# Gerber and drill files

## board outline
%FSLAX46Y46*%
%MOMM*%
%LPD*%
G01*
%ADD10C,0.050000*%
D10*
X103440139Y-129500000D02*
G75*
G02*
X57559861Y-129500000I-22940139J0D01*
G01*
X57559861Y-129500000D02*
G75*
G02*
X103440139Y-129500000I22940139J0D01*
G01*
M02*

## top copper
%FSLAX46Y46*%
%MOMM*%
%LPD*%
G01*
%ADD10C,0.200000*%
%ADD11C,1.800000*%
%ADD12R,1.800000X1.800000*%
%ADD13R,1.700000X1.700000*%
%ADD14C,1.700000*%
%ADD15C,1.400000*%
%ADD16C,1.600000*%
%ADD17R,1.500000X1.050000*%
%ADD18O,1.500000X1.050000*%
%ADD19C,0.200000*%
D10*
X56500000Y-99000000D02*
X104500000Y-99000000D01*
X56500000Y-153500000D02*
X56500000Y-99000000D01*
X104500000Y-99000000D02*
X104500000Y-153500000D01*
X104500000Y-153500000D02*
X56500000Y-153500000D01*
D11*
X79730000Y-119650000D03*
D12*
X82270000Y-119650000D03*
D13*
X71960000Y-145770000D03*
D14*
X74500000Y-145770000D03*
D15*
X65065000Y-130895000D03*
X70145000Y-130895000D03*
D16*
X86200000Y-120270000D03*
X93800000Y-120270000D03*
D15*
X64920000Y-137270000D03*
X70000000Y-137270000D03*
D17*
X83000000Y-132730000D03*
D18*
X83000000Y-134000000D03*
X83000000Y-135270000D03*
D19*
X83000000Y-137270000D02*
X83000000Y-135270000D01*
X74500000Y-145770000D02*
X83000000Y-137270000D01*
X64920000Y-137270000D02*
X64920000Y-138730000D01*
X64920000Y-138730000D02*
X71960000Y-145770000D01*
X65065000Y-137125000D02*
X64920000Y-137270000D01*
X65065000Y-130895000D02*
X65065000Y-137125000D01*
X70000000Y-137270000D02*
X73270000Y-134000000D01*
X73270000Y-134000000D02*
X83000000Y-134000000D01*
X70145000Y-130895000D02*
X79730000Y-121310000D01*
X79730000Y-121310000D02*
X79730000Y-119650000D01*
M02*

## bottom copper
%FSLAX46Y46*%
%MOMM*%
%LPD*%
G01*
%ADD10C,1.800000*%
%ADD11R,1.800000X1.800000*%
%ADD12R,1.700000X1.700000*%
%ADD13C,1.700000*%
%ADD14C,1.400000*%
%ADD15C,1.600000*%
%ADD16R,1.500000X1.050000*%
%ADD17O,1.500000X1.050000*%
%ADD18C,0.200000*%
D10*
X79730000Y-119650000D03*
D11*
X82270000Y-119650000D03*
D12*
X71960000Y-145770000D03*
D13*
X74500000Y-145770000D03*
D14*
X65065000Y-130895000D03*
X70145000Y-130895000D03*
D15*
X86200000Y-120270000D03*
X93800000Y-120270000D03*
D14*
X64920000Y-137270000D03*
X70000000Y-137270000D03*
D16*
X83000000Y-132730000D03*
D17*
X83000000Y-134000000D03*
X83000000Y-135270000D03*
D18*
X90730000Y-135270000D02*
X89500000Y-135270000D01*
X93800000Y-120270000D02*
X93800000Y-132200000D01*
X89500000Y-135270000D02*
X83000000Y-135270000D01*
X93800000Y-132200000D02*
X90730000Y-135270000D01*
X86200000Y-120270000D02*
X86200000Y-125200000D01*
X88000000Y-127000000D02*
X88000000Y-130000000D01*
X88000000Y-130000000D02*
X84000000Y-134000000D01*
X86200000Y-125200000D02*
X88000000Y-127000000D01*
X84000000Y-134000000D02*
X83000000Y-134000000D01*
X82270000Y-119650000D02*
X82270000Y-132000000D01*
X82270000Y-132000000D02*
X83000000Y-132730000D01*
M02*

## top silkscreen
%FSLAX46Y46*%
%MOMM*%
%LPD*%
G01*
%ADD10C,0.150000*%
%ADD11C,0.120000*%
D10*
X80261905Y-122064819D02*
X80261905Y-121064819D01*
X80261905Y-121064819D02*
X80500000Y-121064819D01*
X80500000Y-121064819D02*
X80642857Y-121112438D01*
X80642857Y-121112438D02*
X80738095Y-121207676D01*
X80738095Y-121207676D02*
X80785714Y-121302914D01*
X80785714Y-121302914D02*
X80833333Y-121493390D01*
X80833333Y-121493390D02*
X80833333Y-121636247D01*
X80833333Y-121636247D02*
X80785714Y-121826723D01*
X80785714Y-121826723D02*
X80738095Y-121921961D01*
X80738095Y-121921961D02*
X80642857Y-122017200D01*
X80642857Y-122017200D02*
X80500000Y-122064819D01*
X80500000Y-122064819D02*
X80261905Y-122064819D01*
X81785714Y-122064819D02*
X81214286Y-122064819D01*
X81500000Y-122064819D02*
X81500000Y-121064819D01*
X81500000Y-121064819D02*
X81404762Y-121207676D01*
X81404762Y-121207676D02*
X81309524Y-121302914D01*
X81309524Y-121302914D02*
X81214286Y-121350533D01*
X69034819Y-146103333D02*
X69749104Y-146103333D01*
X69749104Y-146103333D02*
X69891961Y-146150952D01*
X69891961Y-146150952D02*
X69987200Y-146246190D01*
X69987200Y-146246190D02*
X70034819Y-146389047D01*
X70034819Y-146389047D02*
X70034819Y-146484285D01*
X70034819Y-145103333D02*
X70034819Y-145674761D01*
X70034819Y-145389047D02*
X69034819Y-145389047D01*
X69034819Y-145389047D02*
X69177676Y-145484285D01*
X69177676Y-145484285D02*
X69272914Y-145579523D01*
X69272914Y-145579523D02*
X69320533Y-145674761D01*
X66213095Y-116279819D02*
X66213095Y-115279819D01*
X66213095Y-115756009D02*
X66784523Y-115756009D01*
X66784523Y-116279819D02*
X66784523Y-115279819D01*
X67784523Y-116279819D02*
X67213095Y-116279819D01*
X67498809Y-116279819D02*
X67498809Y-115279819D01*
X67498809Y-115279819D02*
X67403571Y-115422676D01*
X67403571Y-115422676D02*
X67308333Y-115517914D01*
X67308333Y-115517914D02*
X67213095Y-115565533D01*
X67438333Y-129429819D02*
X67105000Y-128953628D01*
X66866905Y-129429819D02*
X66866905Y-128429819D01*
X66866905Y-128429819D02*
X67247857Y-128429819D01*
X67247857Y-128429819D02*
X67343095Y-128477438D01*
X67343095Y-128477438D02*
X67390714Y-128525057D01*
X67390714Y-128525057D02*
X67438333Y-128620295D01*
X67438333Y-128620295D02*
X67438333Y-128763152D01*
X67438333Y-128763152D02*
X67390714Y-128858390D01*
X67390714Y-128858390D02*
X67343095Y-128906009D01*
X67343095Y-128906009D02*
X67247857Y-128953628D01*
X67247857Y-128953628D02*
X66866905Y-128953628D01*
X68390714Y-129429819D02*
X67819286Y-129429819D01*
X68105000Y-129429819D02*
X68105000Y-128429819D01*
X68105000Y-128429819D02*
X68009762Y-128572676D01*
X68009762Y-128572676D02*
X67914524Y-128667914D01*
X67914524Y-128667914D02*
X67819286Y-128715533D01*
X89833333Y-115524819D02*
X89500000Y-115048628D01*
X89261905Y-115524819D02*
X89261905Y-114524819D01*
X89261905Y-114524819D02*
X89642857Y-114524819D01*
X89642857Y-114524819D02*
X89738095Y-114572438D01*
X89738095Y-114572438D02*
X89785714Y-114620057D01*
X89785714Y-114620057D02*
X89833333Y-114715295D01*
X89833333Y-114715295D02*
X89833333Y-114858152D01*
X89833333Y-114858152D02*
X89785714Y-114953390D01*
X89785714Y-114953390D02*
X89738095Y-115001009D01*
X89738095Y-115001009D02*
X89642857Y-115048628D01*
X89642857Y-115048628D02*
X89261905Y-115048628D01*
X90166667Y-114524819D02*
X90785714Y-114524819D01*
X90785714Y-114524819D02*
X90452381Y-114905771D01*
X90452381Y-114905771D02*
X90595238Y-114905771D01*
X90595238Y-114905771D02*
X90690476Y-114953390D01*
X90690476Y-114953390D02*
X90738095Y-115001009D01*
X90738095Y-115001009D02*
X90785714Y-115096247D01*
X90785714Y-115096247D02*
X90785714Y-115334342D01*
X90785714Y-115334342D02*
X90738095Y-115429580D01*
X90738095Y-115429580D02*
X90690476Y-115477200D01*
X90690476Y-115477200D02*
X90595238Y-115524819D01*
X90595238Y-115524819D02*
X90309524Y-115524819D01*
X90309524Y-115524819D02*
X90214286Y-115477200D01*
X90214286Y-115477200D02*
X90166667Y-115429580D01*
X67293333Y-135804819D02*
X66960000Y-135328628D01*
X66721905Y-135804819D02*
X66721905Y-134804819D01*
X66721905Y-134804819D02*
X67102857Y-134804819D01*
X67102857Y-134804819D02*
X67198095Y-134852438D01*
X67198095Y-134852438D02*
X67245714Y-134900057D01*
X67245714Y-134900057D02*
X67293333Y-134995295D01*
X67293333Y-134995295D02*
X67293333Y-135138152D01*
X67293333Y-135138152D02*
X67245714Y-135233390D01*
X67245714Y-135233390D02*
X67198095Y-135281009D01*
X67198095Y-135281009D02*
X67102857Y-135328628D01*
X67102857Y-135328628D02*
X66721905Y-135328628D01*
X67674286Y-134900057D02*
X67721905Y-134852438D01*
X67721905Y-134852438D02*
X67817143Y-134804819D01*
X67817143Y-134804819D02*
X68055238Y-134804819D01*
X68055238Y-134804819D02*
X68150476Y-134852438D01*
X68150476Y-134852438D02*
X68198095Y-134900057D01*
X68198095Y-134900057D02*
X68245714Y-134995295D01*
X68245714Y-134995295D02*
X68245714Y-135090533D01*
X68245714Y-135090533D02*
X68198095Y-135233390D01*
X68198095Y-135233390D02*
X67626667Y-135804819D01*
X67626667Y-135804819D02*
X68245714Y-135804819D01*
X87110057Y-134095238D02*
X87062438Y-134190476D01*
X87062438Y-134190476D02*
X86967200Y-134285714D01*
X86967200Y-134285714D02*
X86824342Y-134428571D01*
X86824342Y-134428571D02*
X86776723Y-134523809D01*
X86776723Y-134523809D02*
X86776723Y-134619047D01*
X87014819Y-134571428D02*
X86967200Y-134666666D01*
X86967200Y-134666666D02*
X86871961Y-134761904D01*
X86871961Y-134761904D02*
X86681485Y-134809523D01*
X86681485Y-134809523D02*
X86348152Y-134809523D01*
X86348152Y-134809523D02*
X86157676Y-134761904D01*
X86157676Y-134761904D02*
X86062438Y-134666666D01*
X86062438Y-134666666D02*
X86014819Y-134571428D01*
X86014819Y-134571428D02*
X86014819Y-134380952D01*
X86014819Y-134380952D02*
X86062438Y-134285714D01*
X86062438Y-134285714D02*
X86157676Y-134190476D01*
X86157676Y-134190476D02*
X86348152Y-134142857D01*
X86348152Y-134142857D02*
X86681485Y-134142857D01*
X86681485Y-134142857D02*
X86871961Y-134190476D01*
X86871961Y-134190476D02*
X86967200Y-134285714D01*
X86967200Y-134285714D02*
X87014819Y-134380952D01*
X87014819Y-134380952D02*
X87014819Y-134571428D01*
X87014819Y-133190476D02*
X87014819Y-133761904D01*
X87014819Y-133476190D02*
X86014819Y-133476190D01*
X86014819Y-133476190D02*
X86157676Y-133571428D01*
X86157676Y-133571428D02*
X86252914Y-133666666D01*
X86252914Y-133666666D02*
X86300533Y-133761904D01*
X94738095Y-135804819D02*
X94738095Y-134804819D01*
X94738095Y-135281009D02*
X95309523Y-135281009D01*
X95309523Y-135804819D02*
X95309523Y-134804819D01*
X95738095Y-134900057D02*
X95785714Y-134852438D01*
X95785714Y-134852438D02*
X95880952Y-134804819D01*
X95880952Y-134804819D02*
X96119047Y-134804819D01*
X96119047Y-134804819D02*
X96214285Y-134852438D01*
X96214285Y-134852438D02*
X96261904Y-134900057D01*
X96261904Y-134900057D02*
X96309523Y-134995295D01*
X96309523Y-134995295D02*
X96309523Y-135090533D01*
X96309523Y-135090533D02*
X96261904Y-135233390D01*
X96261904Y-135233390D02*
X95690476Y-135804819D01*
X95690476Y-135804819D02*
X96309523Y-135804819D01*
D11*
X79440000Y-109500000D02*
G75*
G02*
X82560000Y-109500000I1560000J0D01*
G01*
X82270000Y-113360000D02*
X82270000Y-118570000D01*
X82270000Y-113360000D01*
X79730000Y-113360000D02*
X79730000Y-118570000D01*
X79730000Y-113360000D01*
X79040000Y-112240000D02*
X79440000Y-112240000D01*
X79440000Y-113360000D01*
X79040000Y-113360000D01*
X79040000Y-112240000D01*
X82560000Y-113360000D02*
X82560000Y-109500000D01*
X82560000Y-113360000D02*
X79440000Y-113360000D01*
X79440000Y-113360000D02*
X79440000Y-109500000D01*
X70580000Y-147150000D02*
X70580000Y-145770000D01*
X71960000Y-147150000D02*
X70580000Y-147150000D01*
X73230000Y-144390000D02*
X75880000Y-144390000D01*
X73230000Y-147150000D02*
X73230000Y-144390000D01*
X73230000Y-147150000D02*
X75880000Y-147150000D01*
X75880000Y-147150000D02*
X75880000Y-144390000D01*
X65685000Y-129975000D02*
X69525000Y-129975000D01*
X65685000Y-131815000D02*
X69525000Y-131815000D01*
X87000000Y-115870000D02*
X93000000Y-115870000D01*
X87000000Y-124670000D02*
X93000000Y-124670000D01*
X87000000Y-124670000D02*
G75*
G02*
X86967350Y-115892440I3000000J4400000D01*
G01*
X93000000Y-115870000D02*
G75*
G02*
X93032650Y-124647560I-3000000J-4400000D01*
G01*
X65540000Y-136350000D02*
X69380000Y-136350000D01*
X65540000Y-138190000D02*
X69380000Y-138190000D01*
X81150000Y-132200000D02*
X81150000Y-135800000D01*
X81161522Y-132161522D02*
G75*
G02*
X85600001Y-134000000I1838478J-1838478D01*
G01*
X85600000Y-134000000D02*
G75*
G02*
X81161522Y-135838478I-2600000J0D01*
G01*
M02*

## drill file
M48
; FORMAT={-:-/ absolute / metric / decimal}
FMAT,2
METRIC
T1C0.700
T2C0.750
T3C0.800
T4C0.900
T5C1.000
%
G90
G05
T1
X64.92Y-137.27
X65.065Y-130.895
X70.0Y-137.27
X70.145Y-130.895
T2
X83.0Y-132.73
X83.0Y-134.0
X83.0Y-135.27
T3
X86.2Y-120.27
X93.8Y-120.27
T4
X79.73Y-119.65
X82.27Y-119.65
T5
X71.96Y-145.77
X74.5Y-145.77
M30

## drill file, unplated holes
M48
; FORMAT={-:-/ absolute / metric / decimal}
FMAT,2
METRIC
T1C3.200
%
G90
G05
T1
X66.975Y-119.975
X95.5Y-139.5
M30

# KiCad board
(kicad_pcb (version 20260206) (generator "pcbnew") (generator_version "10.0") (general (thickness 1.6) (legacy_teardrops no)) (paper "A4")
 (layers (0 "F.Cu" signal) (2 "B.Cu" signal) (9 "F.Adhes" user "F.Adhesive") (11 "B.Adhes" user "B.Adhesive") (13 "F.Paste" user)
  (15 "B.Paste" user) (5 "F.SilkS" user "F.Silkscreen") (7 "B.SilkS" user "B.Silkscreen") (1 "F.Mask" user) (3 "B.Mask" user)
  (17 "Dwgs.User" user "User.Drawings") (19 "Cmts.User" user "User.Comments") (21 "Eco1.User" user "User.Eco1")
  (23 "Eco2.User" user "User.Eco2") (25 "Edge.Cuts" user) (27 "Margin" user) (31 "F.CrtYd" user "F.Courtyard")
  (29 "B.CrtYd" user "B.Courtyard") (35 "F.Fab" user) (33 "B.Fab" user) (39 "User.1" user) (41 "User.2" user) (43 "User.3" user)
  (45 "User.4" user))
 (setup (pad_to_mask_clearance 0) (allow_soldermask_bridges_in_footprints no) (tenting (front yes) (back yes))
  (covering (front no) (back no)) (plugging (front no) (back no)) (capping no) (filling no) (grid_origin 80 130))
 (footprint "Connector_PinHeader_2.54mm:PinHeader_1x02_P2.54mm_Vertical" (layer "F.Cu") (at 71.96 145.77 90)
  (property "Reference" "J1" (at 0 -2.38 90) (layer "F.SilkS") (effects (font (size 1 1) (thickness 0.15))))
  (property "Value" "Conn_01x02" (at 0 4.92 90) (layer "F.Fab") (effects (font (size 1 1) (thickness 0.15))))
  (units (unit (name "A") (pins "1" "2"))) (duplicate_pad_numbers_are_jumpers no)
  (fp_line (start -1.38 -1.38) (end 0 -1.38) (stroke (width 0.12) (type solid)) (layer "F.SilkS"))
  (fp_line (start -1.38 0) (end -1.38 -1.38) (stroke (width 0.12) (type solid)) (layer "F.SilkS"))
  (fp_line (start 1.38 1.27) (end 1.38 3.92) (stroke (width 0.12) (type solid)) (layer "F.SilkS"))
  (fp_line (start -1.38 1.27) (end 1.38 1.27) (stroke (width 0.12) (type solid)) (layer "F.SilkS"))
  (fp_line (start -1.38 1.27) (end -1.38 3.92) (stroke (width 0.12) (type solid)) (layer "F.SilkS"))
  (fp_line (start -1.38 3.92) (end 1.38 3.92) (stroke (width 0.12) (type solid)) (layer "F.SilkS"))
  (pad "1" thru_hole rect (at 0 0 90) (size 1.7 1.7) (drill 1) (layers "*.Cu" "*.Mask") (remove_unused_layers no) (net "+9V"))
  (pad "2" thru_hole circle (at 0 2.54 90) (size 1.7 1.7) (drill 1) (layers "*.Cu" "*.Mask") (remove_unused_layers no) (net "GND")))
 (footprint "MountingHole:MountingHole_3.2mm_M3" (layer "F.Cu") (at 66.975 119.975)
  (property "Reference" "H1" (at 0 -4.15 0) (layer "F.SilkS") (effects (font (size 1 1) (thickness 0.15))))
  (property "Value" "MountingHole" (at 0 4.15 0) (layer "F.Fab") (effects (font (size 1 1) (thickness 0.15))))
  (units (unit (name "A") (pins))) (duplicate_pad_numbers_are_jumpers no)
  (pad "" np_thru_hole circle (at 0 0) (size 3.2 3.2) (drill 3.2) (layers "*.Cu" "*.Mask")))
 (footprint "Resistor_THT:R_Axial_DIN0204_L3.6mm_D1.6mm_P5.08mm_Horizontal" (layer "F.Cu") (at 65.065 130.895)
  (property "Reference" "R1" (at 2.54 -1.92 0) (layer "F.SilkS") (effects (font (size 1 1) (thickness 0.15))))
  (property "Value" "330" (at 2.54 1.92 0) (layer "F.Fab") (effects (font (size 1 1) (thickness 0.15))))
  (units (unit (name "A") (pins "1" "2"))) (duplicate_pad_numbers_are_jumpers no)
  (fp_line (start 0.62 -0.92) (end 4.46 -0.92) (stroke (width 0.12) (type solid)) (layer "F.SilkS"))
  (fp_line (start 0.62 0.92) (end 4.46 0.92) (stroke (width 0.12) (type solid)) (layer "F.SilkS"))
  (pad "1" thru_hole circle (at 0 0) (size 1.4 1.4) (drill 0.7) (layers "*.Cu" "*.Mask") (remove_unused_layers no) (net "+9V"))
  (pad "2" thru_hole circle (at 5.08 0) (size 1.4 1.4) (drill 0.7) (layers "*.Cu" "*.Mask") (remove_unused_layers no) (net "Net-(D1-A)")))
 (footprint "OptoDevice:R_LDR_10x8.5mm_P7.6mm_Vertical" (layer "F.Cu") (at 86.2 120.27)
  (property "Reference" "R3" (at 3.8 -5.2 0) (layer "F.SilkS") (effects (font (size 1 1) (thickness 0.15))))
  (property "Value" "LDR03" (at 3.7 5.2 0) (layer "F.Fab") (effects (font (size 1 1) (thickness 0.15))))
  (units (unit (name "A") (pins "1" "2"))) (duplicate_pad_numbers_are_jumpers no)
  (fp_line (start 0.8 -4.4) (end 6.8 -4.4) (stroke (width 0.12) (type solid)) (layer "F.SilkS"))
  (fp_line (start 0.8 4.4) (end 6.8 4.4) (stroke (width 0.12) (type solid)) (layer "F.SilkS"))
  (fp_arc (start 0.8 4.4) (mid -1.525374 0.019809) (end 0.76735 -4.37756) (stroke (width 0.12) (type solid)) (layer "F.SilkS"))
  (fp_arc (start 6.8 -4.4) (mid 9.125374 -0.019809) (end 6.83265 4.37756) (stroke (width 0.12) (type solid)) (layer "F.SilkS"))
  (pad "1" thru_hole circle (at 0 0) (size 1.6 1.6) (drill 0.8) (layers "*.Cu" "*.Mask") (remove_unused_layers no) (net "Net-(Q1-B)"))
  (pad "2" thru_hole circle (at 7.6 0) (size 1.6 1.6) (drill 0.8) (layers "*.Cu" "*.Mask") (remove_unused_layers no) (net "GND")))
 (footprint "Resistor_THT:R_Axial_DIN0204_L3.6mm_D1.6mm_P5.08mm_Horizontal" (layer "F.Cu") (at 64.92 137.27)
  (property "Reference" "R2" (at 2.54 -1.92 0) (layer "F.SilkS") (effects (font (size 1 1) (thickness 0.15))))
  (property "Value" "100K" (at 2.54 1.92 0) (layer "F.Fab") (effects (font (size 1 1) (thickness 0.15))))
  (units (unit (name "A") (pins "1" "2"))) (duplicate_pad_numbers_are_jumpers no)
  (fp_line (start 0.62 -0.92) (end 4.46 -0.92) (stroke (width 0.12) (type solid)) (layer "F.SilkS"))
  (fp_line (start 0.62 0.92) (end 4.46 0.92) (stroke (width 0.12) (type solid)) (layer "F.SilkS"))
  (pad "1" thru_hole circle (at 0 0) (size 1.4 1.4) (drill 0.7) (layers "*.Cu" "*.Mask") (remove_unused_layers no) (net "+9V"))
  (pad "2" thru_hole circle (at 5.08 0) (size 1.4 1.4) (drill 0.7) (layers "*.Cu" "*.Mask") (remove_unused_layers no) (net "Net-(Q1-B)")))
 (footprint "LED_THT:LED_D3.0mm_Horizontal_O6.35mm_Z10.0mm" (layer "F.Cu") (at 82.27 119.65 180)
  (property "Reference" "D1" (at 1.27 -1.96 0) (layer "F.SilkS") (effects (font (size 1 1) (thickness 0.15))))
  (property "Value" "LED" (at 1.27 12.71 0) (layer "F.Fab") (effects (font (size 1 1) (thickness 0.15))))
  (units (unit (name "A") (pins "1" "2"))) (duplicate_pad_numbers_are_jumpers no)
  (fp_line (start 2.83 6.29) (end 2.83 10.15) (stroke (width 0.12) (type solid)) (layer "F.SilkS"))
  (fp_line (start -0.29 6.29) (end 2.83 6.29) (stroke (width 0.12) (type solid)) (layer "F.SilkS"))
  (fp_line (start -0.29 6.29) (end -0.29 10.15) (stroke (width 0.12) (type solid)) (layer "F.SilkS"))
  (fp_rect (start 2.83 6.29) (end 3.23 7.41) (stroke (width 0.12) (type solid)) (fill no) (layer "F.SilkS"))
  (fp_rect (start 2.54 1.08) (end 2.54 6.29) (stroke (width 0.12) (type solid)) (fill no) (layer "F.SilkS"))
  (fp_rect (start 0 1.08) (end 0 6.29) (stroke (width 0.12) (type solid)) (fill no) (layer "F.SilkS"))
  (fp_arc (start 2.83 10.15) (mid 1.27 11.71) (end -0.29 10.15) (stroke (width 0.12) (type solid)) (layer "F.SilkS"))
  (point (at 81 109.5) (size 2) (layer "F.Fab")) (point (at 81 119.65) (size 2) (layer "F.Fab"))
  (pad "1" thru_hole rect (at 0 0 180) (size 1.8 1.8) (drill 0.9) (layers "*.Cu" "*.Mask") (remove_unused_layers no) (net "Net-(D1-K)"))
  (pad "2" thru_hole circle (at 2.54 0 180) (size 1.8 1.8) (drill 0.9) (layers "*.Cu" "*.Mask") (remove_unused_layers no) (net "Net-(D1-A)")))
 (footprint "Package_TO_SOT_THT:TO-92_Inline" (layer "F.Cu") (at 83 132.73 -90)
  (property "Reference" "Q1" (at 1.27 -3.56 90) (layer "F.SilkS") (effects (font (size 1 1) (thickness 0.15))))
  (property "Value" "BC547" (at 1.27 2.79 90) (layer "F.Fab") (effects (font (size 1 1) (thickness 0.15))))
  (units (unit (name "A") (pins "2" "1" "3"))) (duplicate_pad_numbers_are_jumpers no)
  (fp_line (start -0.53 1.85) (end 3.07 1.85) (stroke (width 0.12) (type solid)) (layer "F.SilkS"))
  (fp_arc (start -0.568478 1.838478) (mid -1.132087 -0.994977) (end 1.27 -2.6) (stroke (width 0.12) (type solid)) (layer "F.SilkS"))
  (fp_arc (start 1.27 -2.6) (mid 3.672087 -0.994977) (end 3.108478 1.838478) (stroke (width 0.12) (type solid)) (layer "F.SilkS"))
  (pad "1" thru_hole rect (at 0 0 270) (size 1.05 1.5) (drill 0.75) (layers "*.Cu" "*.Mask") (remove_unused_layers no) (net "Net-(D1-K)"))
  (pad "2" thru_hole oval (at 1.27 0 270) (size 1.05 1.5) (drill 0.75) (layers "*.Cu" "*.Mask") (remove_unused_layers no) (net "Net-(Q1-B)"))
  (pad "3" thru_hole oval (at 2.54 0 270) (size 1.05 1.5) (drill 0.75) (layers "*.Cu" "*.Mask") (remove_unused_layers no) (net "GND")))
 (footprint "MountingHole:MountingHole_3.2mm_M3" (layer "F.Cu") (at 95.5 139.5)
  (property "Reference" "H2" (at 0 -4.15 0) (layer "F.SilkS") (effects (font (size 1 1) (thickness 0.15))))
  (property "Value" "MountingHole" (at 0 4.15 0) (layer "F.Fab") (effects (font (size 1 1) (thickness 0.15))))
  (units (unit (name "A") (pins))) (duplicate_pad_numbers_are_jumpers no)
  (pad "" np_thru_hole circle (at 0 0) (size 3.2 3.2) (drill 3.2) (layers "*.Cu" "*.Mask")))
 (gr_line (start 56.5 99) (end 104.5 99) (stroke (width 0.2) (type default)) (layer "F.Cu"))
 (gr_line (start 56.5 153.5) (end 56.5 99) (stroke (width 0.2) (type default)) (layer "F.Cu"))
 (gr_line (start 104.5 99) (end 104.5 153.5) (stroke (width 0.2) (type default)) (layer "F.Cu"))
 (gr_circle (center 80.5 129.5) (end 102.5 136) (stroke (width 0.05) (type default)) (fill no) (layer "Edge.Cuts"))
 (segment (start 64.92 137.27) (end 64.92 138.73) (width 0.2) (layer "F.Cu") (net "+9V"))
 (segment (start 64.92 138.73) (end 71.96 145.77) (width 0.2) (layer "F.Cu") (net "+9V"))
 (segment (start 65.065 137.125) (end 64.92 137.27) (width 0.2) (layer "F.Cu") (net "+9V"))
 (segment (start 65.065 130.895) (end 65.065 137.125) (width 0.2) (layer "F.Cu") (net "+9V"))
 (segment (start 83 137.27) (end 83 135.27) (width 0.2) (layer "F.Cu") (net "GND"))
 (segment (start 74.5 145.77) (end 83 137.27) (width 0.2) (layer "F.Cu") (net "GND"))
 (segment (start 90.73 135.27) (end 89.5 135.27) (width 0.2) (layer "B.Cu") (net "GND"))
 (segment (start 93.8 120.27) (end 93.8 132.2) (width 0.2) (layer "B.Cu") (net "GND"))
 (segment (start 89.5 135.27) (end 83 135.27) (width 0.2) (layer "B.Cu") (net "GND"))
 (segment (start 93.8 132.2) (end 90.73 135.27) (width 0.2) (layer "B.Cu") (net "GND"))
 (segment (start 79.73 121.31) (end 79.73 119.65) (width 0.2) (layer "F.Cu") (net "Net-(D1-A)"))
 (segment (start 70.145 130.895) (end 79.73 121.31) (width 0.2) (layer "F.Cu") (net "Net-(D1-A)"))
 (segment (start 70 137.27) (end 73.27 134) (width 0.2) (layer "F.Cu") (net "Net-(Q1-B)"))
 (segment (start 73.27 134) (end 83 134) (width 0.2) (layer "F.Cu") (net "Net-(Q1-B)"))
 (segment (start 86.2 120.27) (end 86.2 125.2) (width 0.2) (layer "B.Cu") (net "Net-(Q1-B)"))
 (segment (start 88 127) (end 88 130) (width 0.2) (layer "B.Cu") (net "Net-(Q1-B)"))
 (segment (start 88 130) (end 84 134) (width 0.2) (layer "B.Cu") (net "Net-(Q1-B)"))
 (segment (start 86.2 125.2) (end 88 127) (width 0.2) (layer "B.Cu") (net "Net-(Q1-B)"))
 (segment (start 84 134) (end 83 134) (width 0.2) (layer "B.Cu") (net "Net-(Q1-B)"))
 (segment (start 82.27 132) (end 83 132.73) (width 0.2) (layer "B.Cu") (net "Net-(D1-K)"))
 (segment (start 82.27 119.65) (end 82.27 132) (width 0.2) (layer "B.Cu") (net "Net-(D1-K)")))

